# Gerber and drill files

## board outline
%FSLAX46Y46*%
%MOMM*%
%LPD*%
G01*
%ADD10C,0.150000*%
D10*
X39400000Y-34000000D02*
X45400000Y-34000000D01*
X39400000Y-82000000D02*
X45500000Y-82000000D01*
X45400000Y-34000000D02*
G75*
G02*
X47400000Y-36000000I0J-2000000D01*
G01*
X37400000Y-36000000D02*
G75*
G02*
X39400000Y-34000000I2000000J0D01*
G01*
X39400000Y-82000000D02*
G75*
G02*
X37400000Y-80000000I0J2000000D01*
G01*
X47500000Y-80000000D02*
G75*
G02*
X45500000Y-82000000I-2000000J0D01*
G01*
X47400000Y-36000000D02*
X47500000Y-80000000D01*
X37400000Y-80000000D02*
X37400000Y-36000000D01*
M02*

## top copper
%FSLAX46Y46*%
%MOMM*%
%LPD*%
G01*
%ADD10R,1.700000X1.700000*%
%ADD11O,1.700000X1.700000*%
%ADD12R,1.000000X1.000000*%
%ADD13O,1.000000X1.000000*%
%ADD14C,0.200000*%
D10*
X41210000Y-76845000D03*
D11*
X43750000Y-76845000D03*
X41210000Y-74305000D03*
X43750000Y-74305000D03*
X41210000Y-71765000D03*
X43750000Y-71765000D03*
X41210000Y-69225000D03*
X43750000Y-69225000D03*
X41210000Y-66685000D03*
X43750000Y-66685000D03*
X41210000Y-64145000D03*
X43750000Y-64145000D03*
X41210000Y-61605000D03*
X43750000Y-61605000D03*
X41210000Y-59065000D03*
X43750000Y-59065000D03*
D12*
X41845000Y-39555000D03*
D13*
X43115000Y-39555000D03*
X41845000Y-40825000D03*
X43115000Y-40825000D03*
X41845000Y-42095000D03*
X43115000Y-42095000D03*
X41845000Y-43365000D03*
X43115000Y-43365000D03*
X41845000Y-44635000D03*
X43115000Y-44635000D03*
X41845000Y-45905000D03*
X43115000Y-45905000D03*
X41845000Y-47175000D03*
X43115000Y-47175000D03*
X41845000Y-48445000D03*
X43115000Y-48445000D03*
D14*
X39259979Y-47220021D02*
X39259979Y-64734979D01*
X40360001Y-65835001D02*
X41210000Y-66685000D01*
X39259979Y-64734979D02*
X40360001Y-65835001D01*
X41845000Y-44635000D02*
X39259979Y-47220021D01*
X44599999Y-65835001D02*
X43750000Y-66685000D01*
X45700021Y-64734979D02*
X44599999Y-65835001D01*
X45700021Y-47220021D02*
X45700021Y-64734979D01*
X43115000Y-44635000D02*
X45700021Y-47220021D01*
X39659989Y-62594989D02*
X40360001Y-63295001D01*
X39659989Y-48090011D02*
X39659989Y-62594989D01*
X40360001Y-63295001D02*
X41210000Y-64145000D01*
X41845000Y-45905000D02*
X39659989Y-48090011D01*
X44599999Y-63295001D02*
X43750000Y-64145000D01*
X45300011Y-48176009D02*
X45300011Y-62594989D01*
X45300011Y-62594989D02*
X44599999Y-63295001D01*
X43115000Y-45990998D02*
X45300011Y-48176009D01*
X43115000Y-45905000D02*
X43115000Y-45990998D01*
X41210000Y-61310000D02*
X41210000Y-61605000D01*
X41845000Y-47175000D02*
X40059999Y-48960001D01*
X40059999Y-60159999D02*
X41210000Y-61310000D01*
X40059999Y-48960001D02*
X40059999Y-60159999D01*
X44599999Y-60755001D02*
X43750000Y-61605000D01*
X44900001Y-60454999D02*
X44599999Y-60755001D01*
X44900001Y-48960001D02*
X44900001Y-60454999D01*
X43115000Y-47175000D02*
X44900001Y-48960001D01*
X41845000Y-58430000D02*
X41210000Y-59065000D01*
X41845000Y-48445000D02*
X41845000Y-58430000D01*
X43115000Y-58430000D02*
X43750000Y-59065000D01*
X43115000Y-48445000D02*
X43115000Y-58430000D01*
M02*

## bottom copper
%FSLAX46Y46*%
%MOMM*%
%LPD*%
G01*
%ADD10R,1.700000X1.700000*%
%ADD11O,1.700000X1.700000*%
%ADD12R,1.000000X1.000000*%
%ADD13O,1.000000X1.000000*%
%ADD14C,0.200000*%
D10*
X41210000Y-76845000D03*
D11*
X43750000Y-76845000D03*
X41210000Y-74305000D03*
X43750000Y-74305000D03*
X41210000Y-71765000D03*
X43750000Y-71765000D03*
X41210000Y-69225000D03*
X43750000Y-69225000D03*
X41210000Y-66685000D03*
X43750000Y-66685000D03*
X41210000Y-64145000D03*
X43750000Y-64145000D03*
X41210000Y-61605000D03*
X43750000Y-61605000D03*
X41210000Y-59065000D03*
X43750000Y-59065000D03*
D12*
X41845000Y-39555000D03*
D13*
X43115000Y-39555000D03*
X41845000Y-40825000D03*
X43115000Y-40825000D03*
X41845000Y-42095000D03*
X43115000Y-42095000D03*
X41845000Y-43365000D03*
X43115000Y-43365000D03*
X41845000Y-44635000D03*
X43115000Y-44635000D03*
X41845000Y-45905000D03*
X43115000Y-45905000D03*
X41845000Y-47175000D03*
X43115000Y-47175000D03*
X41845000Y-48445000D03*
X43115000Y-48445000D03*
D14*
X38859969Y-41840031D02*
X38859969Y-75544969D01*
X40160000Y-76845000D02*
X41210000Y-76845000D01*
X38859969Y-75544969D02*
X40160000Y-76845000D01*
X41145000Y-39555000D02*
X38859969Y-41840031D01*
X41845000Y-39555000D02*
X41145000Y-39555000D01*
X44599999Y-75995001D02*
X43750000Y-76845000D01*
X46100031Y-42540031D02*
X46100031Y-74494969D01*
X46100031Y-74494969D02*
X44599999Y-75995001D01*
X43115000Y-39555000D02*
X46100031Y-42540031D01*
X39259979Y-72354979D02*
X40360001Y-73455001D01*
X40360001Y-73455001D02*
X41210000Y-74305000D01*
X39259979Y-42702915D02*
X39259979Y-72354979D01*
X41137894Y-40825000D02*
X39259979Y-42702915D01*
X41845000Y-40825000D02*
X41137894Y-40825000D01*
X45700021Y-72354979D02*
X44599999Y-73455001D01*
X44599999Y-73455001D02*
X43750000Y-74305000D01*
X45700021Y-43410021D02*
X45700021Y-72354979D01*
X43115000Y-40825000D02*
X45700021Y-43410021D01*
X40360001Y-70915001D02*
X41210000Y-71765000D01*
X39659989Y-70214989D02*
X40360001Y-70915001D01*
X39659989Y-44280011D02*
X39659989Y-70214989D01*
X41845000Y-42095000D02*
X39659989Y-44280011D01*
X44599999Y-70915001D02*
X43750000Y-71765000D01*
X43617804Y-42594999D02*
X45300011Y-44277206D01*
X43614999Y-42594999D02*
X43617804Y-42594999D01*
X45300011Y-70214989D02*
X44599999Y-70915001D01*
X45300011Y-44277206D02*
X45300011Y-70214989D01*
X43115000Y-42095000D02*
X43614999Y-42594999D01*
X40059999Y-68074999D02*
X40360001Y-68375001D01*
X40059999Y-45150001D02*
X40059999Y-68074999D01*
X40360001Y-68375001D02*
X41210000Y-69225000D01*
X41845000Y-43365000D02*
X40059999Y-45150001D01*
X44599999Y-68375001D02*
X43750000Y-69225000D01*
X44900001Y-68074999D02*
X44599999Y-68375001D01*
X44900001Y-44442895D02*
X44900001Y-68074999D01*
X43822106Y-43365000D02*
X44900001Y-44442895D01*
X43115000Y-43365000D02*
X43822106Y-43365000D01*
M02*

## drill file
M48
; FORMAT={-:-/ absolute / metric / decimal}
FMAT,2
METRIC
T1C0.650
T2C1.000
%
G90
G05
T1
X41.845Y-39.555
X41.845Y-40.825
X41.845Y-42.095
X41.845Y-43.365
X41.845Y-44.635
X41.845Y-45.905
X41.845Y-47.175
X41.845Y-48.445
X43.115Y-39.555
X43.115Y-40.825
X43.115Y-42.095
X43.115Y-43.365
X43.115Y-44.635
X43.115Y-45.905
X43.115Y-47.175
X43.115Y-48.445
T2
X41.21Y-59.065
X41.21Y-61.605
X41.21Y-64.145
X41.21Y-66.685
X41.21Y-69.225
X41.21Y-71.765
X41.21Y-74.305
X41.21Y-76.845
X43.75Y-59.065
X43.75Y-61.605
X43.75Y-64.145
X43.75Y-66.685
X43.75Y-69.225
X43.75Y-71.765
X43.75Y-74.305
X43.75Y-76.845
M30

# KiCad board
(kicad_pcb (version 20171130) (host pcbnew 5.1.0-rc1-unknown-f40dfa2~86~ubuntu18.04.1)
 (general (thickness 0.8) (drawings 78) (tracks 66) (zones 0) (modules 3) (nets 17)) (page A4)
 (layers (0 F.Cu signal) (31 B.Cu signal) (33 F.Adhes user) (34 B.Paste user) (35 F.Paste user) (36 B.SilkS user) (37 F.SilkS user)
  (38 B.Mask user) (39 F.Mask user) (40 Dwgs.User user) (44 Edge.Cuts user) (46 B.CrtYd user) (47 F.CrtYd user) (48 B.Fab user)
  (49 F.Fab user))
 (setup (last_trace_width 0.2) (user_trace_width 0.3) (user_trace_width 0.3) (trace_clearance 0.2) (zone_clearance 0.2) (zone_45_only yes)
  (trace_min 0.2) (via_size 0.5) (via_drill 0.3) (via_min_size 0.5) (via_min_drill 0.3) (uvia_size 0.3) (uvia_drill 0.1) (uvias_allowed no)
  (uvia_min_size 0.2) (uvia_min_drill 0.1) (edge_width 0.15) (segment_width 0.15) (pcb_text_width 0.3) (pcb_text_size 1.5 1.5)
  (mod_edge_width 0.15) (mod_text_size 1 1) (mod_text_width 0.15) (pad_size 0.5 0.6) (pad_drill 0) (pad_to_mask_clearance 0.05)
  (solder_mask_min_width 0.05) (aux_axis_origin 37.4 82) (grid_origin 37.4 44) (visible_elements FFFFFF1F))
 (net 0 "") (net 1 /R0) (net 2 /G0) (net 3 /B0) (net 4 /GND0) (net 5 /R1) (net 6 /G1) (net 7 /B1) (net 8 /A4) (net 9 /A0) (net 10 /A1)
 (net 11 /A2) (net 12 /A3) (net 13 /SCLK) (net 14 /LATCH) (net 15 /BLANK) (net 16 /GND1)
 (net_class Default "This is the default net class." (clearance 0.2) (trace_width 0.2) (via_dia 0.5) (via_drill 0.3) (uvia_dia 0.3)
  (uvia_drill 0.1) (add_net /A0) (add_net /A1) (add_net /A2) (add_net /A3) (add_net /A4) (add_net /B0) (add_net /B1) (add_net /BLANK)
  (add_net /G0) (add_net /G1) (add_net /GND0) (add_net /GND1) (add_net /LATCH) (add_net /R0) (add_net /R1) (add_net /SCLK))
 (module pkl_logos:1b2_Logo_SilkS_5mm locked (layer B.Cu) (at 42.109884 54.5)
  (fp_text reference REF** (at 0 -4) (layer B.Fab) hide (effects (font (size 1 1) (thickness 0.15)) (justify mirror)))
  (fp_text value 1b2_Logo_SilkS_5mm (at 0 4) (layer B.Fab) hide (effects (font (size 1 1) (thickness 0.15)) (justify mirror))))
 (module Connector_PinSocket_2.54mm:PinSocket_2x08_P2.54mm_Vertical (layer F.Cu) (at 41.21 76.845 180)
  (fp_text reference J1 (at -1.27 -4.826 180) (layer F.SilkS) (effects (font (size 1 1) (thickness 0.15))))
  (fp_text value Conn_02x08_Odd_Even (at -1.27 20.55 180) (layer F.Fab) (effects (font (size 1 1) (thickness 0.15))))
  (pad 1 thru_hole rect (at 0 0 180) (size 1.7 1.7) (drill 1) (layers *.Cu *.Mask) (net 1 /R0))
  (pad 2 thru_hole oval (at -2.54 0 180) (size 1.7 1.7) (drill 1) (layers *.Cu *.Mask) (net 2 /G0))
  (pad 3 thru_hole oval (at 0 2.54 180) (size 1.7 1.7) (drill 1) (layers *.Cu *.Mask) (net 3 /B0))
  (pad 4 thru_hole oval (at -2.54 2.54 180) (size 1.7 1.7) (drill 1) (layers *.Cu *.Mask) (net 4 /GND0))
  (pad 5 thru_hole oval (at 0 5.08 180) (size 1.7 1.7) (drill 1) (layers *.Cu *.Mask) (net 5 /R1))
  (pad 6 thru_hole oval (at -2.54 5.08 180) (size 1.7 1.7) (drill 1) (layers *.Cu *.Mask) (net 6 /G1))
  (pad 7 thru_hole oval (at 0 7.62 180) (size 1.7 1.7) (drill 1) (layers *.Cu *.Mask) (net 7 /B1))
  (pad 8 thru_hole oval (at -2.54 7.62 180) (size 1.7 1.7) (drill 1) (layers *.Cu *.Mask) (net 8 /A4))
  (pad 9 thru_hole oval (at 0 10.16 180) (size 1.7 1.7) (drill 1) (layers *.Cu *.Mask) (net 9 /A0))
  (pad 10 thru_hole oval (at -2.54 10.16 180) (size 1.7 1.7) (drill 1) (layers *.Cu *.Mask) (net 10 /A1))
  (pad 11 thru_hole oval (at 0 12.7 180) (size 1.7 1.7) (drill 1) (layers *.Cu *.Mask) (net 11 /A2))
  (pad 12 thru_hole oval (at -2.54 12.7 180) (size 1.7 1.7) (drill 1) (layers *.Cu *.Mask) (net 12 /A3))
  (pad 13 thru_hole oval (at 0 15.24 180) (size 1.7 1.7) (drill 1) (layers *.Cu *.Mask) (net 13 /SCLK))
  (pad 14 thru_hole oval (at -2.54 15.24 180) (size 1.7 1.7) (drill 1) (layers *.Cu *.Mask) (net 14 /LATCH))
  (pad 15 thru_hole oval (at 0 17.78 180) (size 1.7 1.7) (drill 1) (layers *.Cu *.Mask) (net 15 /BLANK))
  (pad 16 thru_hole oval (at -2.54 17.78 180) (size 1.7 1.7) (drill 1) (layers *.Cu *.Mask) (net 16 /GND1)))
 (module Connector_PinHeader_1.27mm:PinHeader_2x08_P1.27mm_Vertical (layer F.Cu) (at 41.845 39.555)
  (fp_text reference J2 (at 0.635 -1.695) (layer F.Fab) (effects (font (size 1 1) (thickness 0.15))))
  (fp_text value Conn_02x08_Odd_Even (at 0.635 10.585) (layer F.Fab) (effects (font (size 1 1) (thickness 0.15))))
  (pad 1 thru_hole rect (at 0 0) (size 1 1) (drill 0.65) (layers *.Cu *.Mask) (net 1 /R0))
  (pad 2 thru_hole oval (at 1.27 0) (size 1 1) (drill 0.65) (layers *.Cu *.Mask) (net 2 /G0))
  (pad 3 thru_hole oval (at 0 1.27) (size 1 1) (drill 0.65) (layers *.Cu *.Mask) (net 3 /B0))
  (pad 4 thru_hole oval (at 1.27 1.27) (size 1 1) (drill 0.65) (layers *.Cu *.Mask) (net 4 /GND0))
  (pad 5 thru_hole oval (at 0 2.54) (size 1 1) (drill 0.65) (layers *.Cu *.Mask) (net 5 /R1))
  (pad 6 thru_hole oval (at 1.27 2.54) (size 1 1) (drill 0.65) (layers *.Cu *.Mask) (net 6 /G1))
  (pad 7 thru_hole oval (at 0 3.81) (size 1 1) (drill 0.65) (layers *.Cu *.Mask) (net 7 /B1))
  (pad 8 thru_hole oval (at 1.27 3.81) (size 1 1) (drill 0.65) (layers *.Cu *.Mask) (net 8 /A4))
  (pad 9 thru_hole oval (at 0 5.08) (size 1 1) (drill 0.65) (layers *.Cu *.Mask) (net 9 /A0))
  (pad 10 thru_hole oval (at 1.27 5.08) (size 1 1) (drill 0.65) (layers *.Cu *.Mask) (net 10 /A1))
  (pad 11 thru_hole oval (at 0 6.35) (size 1 1) (drill 0.65) (layers *.Cu *.Mask) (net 11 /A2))
  (pad 12 thru_hole oval (at 1.27 6.35) (size 1 1) (drill 0.65) (layers *.Cu *.Mask) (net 12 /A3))
  (pad 13 thru_hole oval (at 0 7.62) (size 1 1) (drill 0.65) (layers *.Cu *.Mask) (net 13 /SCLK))
  (pad 14 thru_hole oval (at 1.27 7.62) (size 1 1) (drill 0.65) (layers *.Cu *.Mask) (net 14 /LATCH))
  (pad 15 thru_hole oval (at 0 8.89) (size 1 1) (drill 0.65) (layers *.Cu *.Mask) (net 15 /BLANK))
  (pad 16 thru_hole oval (at 1.27 8.89) (size 1 1) (drill 0.65) (layers *.Cu *.Mask) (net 16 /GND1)))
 (gr_line (start 39.4 34) (end 45.4 34) (layer Edge.Cuts) (width 0.15))
 (gr_line (start 39.4 82) (end 45.5 82) (layer Edge.Cuts) (width 0.15))
 (gr_arc (start 45.4 36) (end 47.4 36) (angle -90) (layer Edge.Cuts) (width 0.15))
 (gr_arc (start 39.4 36) (end 39.4 34) (angle -90) (layer Edge.Cuts) (width 0.15))
 (gr_arc (start 39.4 80) (end 37.4 80) (angle -90) (layer Edge.Cuts) (width 0.15))
 (gr_arc (start 45.5 80) (end 45.5 82) (angle -90) (layer Edge.Cuts) (width 0.15))
 (gr_line (start 47.4 36) (end 47.5 80) (layer Edge.Cuts) (width 0.15))
 (gr_line (start 37.4 80) (end 37.4 36) (layer Edge.Cuts) (width 0.15))
 (segment (start 38.859969 41.840031) (end 38.859969 75.544969) (width 0.2) (layer B.Cu) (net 1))
 (segment (start 40.16 76.845) (end 41.21 76.845) (width 0.2) (layer B.Cu) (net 1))
 (segment (start 38.859969 75.544969) (end 40.16 76.845) (width 0.2) (layer B.Cu) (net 1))
 (segment (start 41.145 39.555) (end 38.859969 41.840031) (width 0.2) (layer B.Cu) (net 1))
 (segment (start 41.845 39.555) (end 41.145 39.555) (width 0.2) (layer B.Cu) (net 1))
 (segment (start 44.599999 75.995001) (end 43.75 76.845) (width 0.2) (layer B.Cu) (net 2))
 (segment (start 46.100031 42.540031) (end 46.100031 74.494969) (width 0.2) (layer B.Cu) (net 2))
 (segment (start 46.100031 74.494969) (end 44.599999 75.995001) (width 0.2) (layer B.Cu) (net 2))
 (segment (start 43.115 39.555) (end 46.100031 42.540031) (width 0.2) (layer B.Cu) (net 2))
 (segment (start 39.259979 72.354979) (end 40.360001 73.455001) (width 0.2) (layer B.Cu) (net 3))
 (segment (start 40.360001 73.455001) (end 41.21 74.305) (width 0.2) (layer B.Cu) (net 3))
 (segment (start 39.259979 42.702915) (end 39.259979 72.354979) (width 0.2) (layer B.Cu) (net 3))
 (segment (start 41.137894 40.825) (end 39.259979 42.702915) (width 0.2) (layer B.Cu) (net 3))
 (segment (start 41.845 40.825) (end 41.137894 40.825) (width 0.2) (layer B.Cu) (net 3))
 (segment (start 45.700021 72.354979) (end 44.599999 73.455001) (width 0.2) (layer B.Cu) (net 4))
 (segment (start 44.599999 73.455001) (end 43.75 74.305) (width 0.2) (layer B.Cu) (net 4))
 (segment (start 45.700021 43.410021) (end 45.700021 72.354979) (width 0.2) (layer B.Cu) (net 4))
 (segment (start 43.115 40.825) (end 45.700021 43.410021) (width 0.2) (layer B.Cu) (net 4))
 (segment (start 40.360001 70.915001) (end 41.21 71.765) (width 0.2) (layer B.Cu) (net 5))
 (segment (start 39.659989 70.214989) (end 40.360001 70.915001) (width 0.2) (layer B.Cu) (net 5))
 (segment (start 39.659989 44.280011) (end 39.659989 70.214989) (width 0.2) (layer B.Cu) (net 5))
 (segment (start 41.845 42.095) (end 39.659989 44.280011) (width 0.2) (layer B.Cu) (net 5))
 (segment (start 44.599999 70.915001) (end 43.75 71.765) (width 0.2) (layer B.Cu) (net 6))
 (segment (start 43.617804 42.594999) (end 45.300011 44.277206) (width 0.2) (layer B.Cu) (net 6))
 (segment (start 43.614999 42.594999) (end 43.617804 42.594999) (width 0.2) (layer B.Cu) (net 6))
 (segment (start 45.300011 70.214989) (end 44.599999 70.915001) (width 0.2) (layer B.Cu) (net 6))
 (segment (start 45.300011 44.277206) (end 45.300011 70.214989) (width 0.2) (layer B.Cu) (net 6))
 (segment (start 43.115 42.095) (end 43.614999 42.594999) (width 0.2) (layer B.Cu) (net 6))
 (segment (start 40.059999 68.074999) (end 40.360001 68.375001) (width 0.2) (layer B.Cu) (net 7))
 (segment (start 40.059999 45.150001) (end 40.059999 68.074999) (width 0.2) (layer B.Cu) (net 7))
 (segment (start 40.360001 68.375001) (end 41.21 69.225) (width 0.2) (layer B.Cu) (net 7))
 (segment (start 41.845 43.365) (end 40.059999 45.150001) (width 0.2) (layer B.Cu) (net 7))
 (segment (start 44.599999 68.375001) (end 43.75 69.225) (width 0.2) (layer B.Cu) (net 8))
 (segment (start 44.900001 68.074999) (end 44.599999 68.375001) (width 0.2) (layer B.Cu) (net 8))
 (segment (start 44.900001 44.442895) (end 44.900001 68.074999) (width 0.2) (layer B.Cu) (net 8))
 (segment (start 43.822106 43.365) (end 44.900001 44.442895) (width 0.2) (layer B.Cu) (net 8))
 (segment (start 43.115 43.365) (end 43.822106 43.365) (width 0.2) (layer B.Cu) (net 8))
 (segment (start 39.259979 47.220021) (end 39.259979 64.734979) (width 0.2) (layer F.Cu) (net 9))
 (segment (start 40.360001 65.835001) (end 41.21 66.685) (width 0.2) (layer F.Cu) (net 9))
 (segment (start 39.259979 64.734979) (end 40.360001 65.835001) (width 0.2) (layer F.Cu) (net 9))
 (segment (start 41.845 44.635) (end 39.259979 47.220021) (width 0.2) (layer F.Cu) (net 9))
 (segment (start 44.599999 65.835001) (end 43.75 66.685) (width 0.2) (layer F.Cu) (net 10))
 (segment (start 45.700021 64.734979) (end 44.599999 65.835001) (width 0.2) (layer F.Cu) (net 10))
 (segment (start 45.700021 47.220021) (end 45.700021 64.734979) (width 0.2) (layer F.Cu) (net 10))
 (segment (start 43.115 44.635) (end 45.700021 47.220021) (width 0.2) (layer F.Cu) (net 10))
 (segment (start 39.659989 62.594989) (end 40.360001 63.295001) (width 0.2) (layer F.Cu) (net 11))
 (segment (start 39.659989 48.090011) (end 39.659989 62.594989) (width 0.2) (layer F.Cu) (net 11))
 (segment (start 40.360001 63.295001) (end 41.21 64.145) (width 0.2) (layer F.Cu) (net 11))
 (segment (start 41.845 45.905) (end 39.659989 48.090011) (width 0.2) (layer F.Cu) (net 11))
 (segment (start 44.599999 63.295001) (end 43.75 64.145) (width 0.2) (layer F.Cu) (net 12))
 (segment (start 45.300011 48.176009) (end 45.300011 62.594989) (width 0.2) (layer F.Cu) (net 12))
 (segment (start 45.300011 62.594989) (end 44.599999 63.295001) (width 0.2) (layer F.Cu) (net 12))
 (segment (start 43.115 45.990998) (end 45.300011 48.176009) (width 0.2) (layer F.Cu) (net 12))
 (segment (start 43.115 45.905) (end 43.115 45.990998) (width 0.2) (layer F.Cu) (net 12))
 (segment (start 41.21 61.31) (end 41.21 61.605) (width 0.2) (layer F.Cu) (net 13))
 (segment (start 41.845 47.175) (end 40.059999 48.960001) (width 0.2) (layer F.Cu) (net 13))
 (segment (start 40.059999 60.159999) (end 41.21 61.31) (width 0.2) (layer F.Cu) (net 13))
 (segment (start 40.059999 48.960001) (end 40.059999 60.159999) (width 0.2) (layer F.Cu) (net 13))
 (segment (start 44.599999 60.755001) (end 43.75 61.605) (width 0.2) (layer F.Cu) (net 14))
 (segment (start 44.900001 60.454999) (end 44.599999 60.755001) (width 0.2) (layer F.Cu) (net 14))
 (segment (start 44.900001 48.960001) (end 44.900001 60.454999) (width 0.2) (layer F.Cu) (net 14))
 (segment (start 43.115 47.175) (end 44.900001 48.960001) (width 0.2) (layer F.Cu) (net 14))
 (segment (start 41.845 58.43) (end 41.21 59.065) (width 0.2) (layer F.Cu) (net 15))
 (segment (start 41.845 48.445) (end 41.845 58.43) (width 0.2) (layer F.Cu) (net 15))
 (segment (start 43.115 58.43) (end 43.75 59.065) (width 0.2) (layer F.Cu) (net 16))
 (segment (start 43.115 48.445) (end 43.115 58.43) (width 0.2) (layer F.Cu) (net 16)))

